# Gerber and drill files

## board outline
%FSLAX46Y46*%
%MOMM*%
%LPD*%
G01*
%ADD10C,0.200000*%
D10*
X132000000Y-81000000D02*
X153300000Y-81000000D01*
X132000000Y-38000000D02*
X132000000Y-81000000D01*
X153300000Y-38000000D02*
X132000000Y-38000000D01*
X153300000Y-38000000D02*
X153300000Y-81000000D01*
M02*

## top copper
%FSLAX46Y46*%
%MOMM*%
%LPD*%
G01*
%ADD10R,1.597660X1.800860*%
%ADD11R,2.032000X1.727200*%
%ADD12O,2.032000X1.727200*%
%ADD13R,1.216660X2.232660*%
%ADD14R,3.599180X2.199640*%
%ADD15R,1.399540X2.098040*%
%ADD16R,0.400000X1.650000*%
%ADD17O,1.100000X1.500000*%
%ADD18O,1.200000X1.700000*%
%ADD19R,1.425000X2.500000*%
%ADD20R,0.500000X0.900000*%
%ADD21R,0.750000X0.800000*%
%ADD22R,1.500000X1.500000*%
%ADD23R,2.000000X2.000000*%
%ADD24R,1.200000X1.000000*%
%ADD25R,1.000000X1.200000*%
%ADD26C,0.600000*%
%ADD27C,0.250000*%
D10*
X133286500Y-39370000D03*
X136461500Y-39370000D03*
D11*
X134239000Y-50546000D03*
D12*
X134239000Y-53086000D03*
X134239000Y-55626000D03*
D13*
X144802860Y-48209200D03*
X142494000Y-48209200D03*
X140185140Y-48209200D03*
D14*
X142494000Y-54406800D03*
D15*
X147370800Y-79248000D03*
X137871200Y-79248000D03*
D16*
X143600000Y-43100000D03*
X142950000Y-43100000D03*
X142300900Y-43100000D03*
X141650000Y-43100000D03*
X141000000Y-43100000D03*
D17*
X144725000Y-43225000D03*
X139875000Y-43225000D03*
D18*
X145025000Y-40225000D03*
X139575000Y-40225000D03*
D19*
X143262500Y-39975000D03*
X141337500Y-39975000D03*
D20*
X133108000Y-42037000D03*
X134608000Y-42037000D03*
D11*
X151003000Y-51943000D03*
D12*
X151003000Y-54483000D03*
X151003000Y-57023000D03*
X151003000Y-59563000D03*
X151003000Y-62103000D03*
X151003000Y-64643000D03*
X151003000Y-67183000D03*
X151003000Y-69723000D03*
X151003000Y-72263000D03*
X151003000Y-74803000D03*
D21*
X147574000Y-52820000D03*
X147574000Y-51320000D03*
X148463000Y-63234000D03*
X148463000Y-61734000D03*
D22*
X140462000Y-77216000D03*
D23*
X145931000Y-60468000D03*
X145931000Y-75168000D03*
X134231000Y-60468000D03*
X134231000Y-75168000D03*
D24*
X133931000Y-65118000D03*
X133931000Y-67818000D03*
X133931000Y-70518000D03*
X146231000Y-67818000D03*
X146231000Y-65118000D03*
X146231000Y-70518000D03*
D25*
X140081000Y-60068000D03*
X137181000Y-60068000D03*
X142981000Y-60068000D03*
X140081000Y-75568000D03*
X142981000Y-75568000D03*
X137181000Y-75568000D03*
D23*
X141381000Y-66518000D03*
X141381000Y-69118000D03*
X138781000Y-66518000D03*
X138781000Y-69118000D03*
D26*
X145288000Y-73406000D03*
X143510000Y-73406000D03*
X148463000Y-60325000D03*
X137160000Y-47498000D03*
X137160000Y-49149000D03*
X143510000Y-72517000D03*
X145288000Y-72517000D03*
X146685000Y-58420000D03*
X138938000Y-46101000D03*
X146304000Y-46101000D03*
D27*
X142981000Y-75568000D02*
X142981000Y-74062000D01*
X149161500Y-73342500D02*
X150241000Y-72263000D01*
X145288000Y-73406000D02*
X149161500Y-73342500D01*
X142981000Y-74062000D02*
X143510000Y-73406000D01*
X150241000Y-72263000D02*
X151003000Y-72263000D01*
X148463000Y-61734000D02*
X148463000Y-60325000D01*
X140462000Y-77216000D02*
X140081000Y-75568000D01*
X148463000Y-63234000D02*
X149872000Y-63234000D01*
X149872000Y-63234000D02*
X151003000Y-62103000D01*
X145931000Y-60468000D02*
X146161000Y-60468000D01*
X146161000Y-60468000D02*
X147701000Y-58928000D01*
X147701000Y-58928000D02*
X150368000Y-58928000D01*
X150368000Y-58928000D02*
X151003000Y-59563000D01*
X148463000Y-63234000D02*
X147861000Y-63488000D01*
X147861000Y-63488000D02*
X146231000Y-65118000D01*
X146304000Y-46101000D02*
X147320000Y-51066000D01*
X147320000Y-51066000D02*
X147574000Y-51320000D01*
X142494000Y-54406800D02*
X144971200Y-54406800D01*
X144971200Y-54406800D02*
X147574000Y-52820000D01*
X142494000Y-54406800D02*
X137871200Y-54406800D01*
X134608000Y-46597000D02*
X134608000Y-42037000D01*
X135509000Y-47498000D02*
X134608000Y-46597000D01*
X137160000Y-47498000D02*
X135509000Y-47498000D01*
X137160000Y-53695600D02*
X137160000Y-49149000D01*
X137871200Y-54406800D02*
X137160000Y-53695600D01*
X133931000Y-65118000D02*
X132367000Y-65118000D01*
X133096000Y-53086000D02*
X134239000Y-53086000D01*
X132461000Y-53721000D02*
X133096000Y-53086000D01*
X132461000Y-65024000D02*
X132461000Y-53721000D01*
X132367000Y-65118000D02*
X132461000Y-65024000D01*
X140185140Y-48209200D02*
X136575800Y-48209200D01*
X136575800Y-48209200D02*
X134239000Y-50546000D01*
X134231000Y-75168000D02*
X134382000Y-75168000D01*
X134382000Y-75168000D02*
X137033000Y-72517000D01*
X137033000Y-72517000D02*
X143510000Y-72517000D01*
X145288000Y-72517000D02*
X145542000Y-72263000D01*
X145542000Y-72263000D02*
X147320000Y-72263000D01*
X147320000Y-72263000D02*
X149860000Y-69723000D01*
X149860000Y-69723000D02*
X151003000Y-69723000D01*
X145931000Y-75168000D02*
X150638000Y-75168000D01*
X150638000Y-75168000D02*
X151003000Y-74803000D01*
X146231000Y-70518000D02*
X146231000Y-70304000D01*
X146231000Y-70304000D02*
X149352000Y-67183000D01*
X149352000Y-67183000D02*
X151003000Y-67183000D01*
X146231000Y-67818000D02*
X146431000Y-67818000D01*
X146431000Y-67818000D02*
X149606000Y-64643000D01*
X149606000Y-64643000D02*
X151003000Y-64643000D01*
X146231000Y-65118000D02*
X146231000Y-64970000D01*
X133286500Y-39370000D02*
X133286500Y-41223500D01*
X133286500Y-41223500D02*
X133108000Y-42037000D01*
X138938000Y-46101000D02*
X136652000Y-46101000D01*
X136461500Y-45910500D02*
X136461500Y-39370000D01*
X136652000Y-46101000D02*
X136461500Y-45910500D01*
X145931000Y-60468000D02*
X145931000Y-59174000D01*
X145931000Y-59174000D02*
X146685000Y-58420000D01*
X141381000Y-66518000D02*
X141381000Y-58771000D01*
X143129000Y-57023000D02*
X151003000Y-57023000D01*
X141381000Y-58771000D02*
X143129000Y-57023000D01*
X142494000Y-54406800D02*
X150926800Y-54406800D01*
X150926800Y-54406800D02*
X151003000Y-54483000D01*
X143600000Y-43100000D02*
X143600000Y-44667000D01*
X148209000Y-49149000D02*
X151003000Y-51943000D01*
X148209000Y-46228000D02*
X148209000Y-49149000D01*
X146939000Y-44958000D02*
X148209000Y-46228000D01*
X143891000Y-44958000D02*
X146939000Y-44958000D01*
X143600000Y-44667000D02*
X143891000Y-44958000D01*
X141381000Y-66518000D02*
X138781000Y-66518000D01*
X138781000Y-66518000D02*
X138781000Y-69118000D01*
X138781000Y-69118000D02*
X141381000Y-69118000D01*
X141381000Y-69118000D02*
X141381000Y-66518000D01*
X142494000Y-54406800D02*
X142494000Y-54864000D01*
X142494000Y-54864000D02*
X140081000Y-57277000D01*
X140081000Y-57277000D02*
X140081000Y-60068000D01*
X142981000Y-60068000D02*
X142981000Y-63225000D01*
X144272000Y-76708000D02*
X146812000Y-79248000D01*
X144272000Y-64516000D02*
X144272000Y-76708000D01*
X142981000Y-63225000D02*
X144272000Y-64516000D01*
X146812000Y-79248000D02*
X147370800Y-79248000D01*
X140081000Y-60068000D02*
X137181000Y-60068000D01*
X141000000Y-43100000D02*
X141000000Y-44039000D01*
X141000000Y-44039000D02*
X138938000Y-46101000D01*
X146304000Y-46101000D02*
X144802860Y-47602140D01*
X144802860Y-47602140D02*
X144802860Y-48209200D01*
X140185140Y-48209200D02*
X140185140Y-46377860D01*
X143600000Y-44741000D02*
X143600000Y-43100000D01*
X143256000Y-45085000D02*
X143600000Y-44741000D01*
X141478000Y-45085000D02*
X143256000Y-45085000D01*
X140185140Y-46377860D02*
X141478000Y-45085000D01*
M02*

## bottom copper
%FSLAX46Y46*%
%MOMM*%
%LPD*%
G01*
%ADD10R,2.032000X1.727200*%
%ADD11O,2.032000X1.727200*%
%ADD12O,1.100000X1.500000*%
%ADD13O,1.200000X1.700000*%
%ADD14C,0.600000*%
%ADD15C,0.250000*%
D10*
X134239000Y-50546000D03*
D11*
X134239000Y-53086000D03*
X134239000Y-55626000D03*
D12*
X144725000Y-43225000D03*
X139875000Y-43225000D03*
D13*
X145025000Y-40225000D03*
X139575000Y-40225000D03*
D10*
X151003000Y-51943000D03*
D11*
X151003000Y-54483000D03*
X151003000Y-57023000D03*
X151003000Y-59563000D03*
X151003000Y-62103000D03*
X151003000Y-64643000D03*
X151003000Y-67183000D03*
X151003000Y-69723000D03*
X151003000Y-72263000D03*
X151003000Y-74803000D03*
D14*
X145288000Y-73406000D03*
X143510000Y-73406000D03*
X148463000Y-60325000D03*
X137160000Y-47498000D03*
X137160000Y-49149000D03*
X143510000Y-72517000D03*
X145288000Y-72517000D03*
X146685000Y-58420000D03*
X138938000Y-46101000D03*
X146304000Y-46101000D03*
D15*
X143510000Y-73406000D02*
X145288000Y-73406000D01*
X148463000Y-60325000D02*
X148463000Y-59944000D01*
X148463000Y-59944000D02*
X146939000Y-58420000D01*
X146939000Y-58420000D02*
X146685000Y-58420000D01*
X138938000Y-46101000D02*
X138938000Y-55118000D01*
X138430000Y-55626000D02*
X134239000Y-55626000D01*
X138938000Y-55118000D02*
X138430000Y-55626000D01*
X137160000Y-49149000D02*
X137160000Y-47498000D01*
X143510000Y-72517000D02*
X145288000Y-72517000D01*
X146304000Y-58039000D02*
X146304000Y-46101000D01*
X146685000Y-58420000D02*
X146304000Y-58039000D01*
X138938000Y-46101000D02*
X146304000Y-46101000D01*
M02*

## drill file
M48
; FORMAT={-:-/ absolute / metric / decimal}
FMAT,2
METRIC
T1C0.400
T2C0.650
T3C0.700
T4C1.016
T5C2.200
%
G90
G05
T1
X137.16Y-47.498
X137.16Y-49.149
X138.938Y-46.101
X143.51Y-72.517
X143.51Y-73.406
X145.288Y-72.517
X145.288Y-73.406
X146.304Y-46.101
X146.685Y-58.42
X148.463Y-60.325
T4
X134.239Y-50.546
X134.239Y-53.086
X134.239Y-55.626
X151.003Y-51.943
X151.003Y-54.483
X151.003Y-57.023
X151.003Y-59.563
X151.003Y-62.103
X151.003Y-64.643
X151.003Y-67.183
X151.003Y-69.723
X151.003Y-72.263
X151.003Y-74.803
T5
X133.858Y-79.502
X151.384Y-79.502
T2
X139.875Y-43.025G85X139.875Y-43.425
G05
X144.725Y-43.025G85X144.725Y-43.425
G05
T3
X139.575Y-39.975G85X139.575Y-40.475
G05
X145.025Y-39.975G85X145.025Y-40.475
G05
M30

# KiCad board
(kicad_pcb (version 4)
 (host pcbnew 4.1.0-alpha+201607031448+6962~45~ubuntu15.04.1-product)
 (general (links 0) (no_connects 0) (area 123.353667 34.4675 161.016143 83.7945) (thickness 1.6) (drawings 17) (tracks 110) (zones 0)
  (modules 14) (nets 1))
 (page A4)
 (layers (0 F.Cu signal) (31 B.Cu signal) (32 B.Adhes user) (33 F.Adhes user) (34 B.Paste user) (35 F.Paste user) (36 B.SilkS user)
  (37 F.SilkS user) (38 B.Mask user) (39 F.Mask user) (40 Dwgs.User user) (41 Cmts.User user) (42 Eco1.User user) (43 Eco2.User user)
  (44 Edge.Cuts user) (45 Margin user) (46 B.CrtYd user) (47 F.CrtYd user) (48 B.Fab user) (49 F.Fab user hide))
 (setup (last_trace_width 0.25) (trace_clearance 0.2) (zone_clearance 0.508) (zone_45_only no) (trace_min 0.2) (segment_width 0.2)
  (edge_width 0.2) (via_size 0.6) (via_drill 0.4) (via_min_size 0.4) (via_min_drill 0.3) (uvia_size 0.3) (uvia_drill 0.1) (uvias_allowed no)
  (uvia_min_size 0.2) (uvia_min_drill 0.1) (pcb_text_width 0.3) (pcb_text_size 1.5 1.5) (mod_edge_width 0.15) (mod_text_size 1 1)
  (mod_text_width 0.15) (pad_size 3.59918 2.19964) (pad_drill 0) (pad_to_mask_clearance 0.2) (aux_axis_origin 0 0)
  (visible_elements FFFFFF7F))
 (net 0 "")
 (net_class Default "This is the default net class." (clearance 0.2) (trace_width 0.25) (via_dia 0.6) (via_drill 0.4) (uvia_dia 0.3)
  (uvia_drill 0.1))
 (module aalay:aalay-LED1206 (layer F.Cu) (at 134.874 39.37)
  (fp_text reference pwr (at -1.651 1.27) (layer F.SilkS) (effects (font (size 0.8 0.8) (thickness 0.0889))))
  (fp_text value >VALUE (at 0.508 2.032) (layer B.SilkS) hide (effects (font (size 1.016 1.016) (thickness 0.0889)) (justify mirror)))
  (pad A smd rect (at -1.5875 0) (size 1.59766 1.80086) (layers F.Cu F.Paste F.Mask))
  (pad K smd rect (at 1.5875 0) (size 1.59766 1.80086) (layers F.Cu F.Paste F.Mask)))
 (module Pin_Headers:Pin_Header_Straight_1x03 (layer F.Cu) (at 134.239 50.546)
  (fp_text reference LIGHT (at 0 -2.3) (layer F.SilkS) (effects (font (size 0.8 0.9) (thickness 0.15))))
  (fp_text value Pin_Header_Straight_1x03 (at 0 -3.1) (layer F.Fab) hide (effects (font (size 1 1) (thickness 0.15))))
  (pad 1 thru_hole rect (at 0 0) (size 2.032 1.7272) (drill 1.016) (layers *.Cu *.Mask F.SilkS))
  (pad 2 thru_hole oval (at 0 2.54) (size 2.032 1.7272) (drill 1.016) (layers *.Cu *.Mask F.SilkS))
  (pad 3 thru_hole oval (at 0 5.08) (size 2.032 1.7272) (drill 1.016) (layers *.Cu *.Mask F.SilkS)))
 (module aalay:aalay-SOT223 (layer F.Cu) (at 142.494 51.308 180)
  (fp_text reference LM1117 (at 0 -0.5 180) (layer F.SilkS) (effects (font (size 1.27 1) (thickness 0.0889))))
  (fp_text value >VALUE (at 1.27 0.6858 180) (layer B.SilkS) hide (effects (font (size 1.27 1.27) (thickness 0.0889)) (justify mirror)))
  (pad GND smd rect (at -2.30886 3.0988 180) (size 1.21666 2.23266) (layers F.Cu F.Paste F.Mask))
  (pad OUT smd rect (at 0 3.0988 180) (size 1.21666 2.23266) (layers F.Cu F.Paste F.Mask))
  (pad IN smd rect (at 2.30886 3.0988 180) (size 1.21666 2.23266) (layers F.Cu F.Paste F.Mask))
  (pad OUT smd rect (at 0 -3.0988 180) (size 3.59918 2.19964) (layers F.Cu F.Paste F.Mask)))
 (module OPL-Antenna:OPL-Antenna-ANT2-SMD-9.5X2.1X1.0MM (layer F.Cu) (at 142.621 79.248 180)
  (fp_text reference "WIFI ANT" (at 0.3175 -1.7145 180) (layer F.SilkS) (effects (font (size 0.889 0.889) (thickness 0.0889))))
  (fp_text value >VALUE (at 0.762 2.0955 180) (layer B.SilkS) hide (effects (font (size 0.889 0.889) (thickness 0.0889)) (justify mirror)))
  (pad 1 smd rect (at -4.7498 0 180) (size 1.39954 2.09804) (layers F.Cu F.Paste F.Mask))
  (pad 2 smd rect (at 4.7498 0 180) (size 1.39954 2.09804) (layers F.Cu F.Paste F.Mask)))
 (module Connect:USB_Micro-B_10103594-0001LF (layer F.Cu) (at 142.3 41.6 180)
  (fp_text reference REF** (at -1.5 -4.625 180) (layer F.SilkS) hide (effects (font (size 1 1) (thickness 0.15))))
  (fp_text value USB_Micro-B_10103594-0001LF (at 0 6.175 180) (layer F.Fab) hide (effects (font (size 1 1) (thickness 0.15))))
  (pad +5 smd rect (at -1.3 -1.5 270) (size 1.65 0.4) (layers F.Cu F.Paste F.Mask))
  (pad D- smd rect (at -0.65 -1.5 270) (size 1.65 0.4) (layers F.Cu F.Paste F.Mask))
  (pad D+ smd rect (at -0.0009 -1.5 270) (size 1.65 0.4) (layers F.Cu F.Paste F.Mask))
  (pad ID smd rect (at 0.65 -1.5 270) (size 1.65 0.4) (layers F.Cu F.Paste F.Mask))
  (pad GND smd rect (at 1.3 -1.5 270) (size 1.65 0.4) (layers F.Cu F.Paste F.Mask))
  (pad 6 thru_hole oval (at -2.425 -1.625 270) (size 1.5 1.1) (drill oval 1.05 0.65) (layers *.Cu *.Mask F.SilkS))
  (pad 6 thru_hole oval (at 2.425 -1.625 270) (size 1.5 1.1) (drill oval 1.05 0.65) (layers *.Cu *.Mask F.SilkS))
  (pad 6 thru_hole oval (at -2.725 1.375 270) (size 1.7 1.2) (drill oval 1.2 0.7) (layers *.Cu *.Mask F.SilkS))
  (pad 6 thru_hole oval (at 2.725 1.375 270) (size 1.7 1.2) (drill oval 1.2 0.7) (layers *.Cu *.Mask F.SilkS))
  (pad 6 smd rect (at -0.9625 1.625 270) (size 2.5 1.425) (layers F.Cu F.Paste F.Mask))
  (pad 6 smd rect (at 0.9625 1.625 270) (size 2.5 1.425) (layers F.Cu F.Paste F.Mask)))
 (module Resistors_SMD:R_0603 (layer F.Cu) (at 133.858 42.037)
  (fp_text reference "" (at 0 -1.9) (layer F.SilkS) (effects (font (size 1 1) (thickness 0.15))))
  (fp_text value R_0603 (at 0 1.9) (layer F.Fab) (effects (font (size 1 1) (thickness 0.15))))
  (pad 1 smd rect (at -0.75 0) (size 0.5 0.9) (layers F.Cu F.Paste F.Mask))
  (pad 2 smd rect (at 0.75 0) (size 0.5 0.9) (layers F.Cu F.Paste F.Mask)))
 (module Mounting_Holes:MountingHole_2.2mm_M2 (layer F.Cu) (at 133.858 79.502)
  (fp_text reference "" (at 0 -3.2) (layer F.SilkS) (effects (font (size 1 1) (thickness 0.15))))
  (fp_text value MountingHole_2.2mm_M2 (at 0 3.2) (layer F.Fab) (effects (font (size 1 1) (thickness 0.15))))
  (pad 1 np_thru_hole circle (at 0 0) (size 2.2 2.2) (drill 2.2) (layers *.Cu *.Mask F.SilkS)))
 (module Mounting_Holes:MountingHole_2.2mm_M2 (layer F.Cu) (at 151.384 79.502)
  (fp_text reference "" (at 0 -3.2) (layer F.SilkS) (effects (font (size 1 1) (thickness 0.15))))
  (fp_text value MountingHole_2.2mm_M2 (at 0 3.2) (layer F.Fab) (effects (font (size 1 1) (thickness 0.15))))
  (pad 1 np_thru_hole circle (at 0 0) (size 2.2 2.2) (drill 2.2) (layers *.Cu *.Mask F.SilkS)))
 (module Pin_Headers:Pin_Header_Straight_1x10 (layer F.Cu) (at 151.003 51.943)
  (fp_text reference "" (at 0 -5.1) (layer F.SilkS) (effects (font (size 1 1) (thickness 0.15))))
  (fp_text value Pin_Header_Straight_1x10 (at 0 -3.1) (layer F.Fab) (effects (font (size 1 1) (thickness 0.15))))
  (pad 1 thru_hole rect (at 0 0) (size 2.032 1.7272) (drill 1.016) (layers *.Cu *.Mask F.SilkS))
  (pad 2 thru_hole oval (at 0 2.54) (size 2.032 1.7272) (drill 1.016) (layers *.Cu *.Mask F.SilkS))
  (pad 3 thru_hole oval (at 0 5.08) (size 2.032 1.7272) (drill 1.016) (layers *.Cu *.Mask F.SilkS))
  (pad 4 thru_hole oval (at 0 7.62) (size 2.032 1.7272) (drill 1.016) (layers *.Cu *.Mask F.SilkS))
  (pad 5 thru_hole oval (at 0 10.16) (size 2.032 1.7272) (drill 1.016) (layers *.Cu *.Mask F.SilkS))
  (pad 6 thru_hole oval (at 0 12.7) (size 2.032 1.7272) (drill 1.016) (layers *.Cu *.Mask F.SilkS))
  (pad 7 thru_hole oval (at 0 15.24) (size 2.032 1.7272) (drill 1.016) (layers *.Cu *.Mask F.SilkS))
  (pad 8 thru_hole oval (at 0 17.78) (size 2.032 1.7272) (drill 1.016) (layers *.Cu *.Mask F.SilkS))
  (pad 9 thru_hole oval (at 0 20.32) (size 2.032 1.7272) (drill 1.016) (layers *.Cu *.Mask F.SilkS))
  (pad 10 thru_hole oval (at 0 22.86) (size 2.032 1.7272) (drill 1.016) (layers *.Cu *.Mask F.SilkS)))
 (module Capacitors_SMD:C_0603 (layer F.Cu) (at 147.574 52.07 90)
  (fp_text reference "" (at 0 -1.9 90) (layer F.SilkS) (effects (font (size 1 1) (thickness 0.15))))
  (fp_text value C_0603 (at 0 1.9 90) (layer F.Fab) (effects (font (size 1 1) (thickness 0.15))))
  (pad 1 smd rect (at -0.75 0 90) (size 0.8 0.75) (layers F.Cu F.Paste F.Mask))
  (pad 2 smd rect (at 0.75 0 90) (size 0.8 0.75) (layers F.Cu F.Paste F.Mask)))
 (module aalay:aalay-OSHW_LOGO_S (layer F.Cu) (at 150.368 44.831)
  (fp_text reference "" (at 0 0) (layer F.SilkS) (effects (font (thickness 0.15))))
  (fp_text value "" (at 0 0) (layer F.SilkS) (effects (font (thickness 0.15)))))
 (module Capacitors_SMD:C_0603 (layer F.Cu) (at 148.463 62.484 90)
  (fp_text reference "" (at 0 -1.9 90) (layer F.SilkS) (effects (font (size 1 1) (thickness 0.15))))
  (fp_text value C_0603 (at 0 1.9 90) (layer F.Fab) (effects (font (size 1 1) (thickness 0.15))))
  (pad 1 smd rect (at -0.75 0 90) (size 0.8 0.75) (layers F.Cu F.Paste F.Mask))
  (pad 2 smd rect (at 0.75 0 90) (size 0.8 0.75) (layers F.Cu F.Paste F.Mask)))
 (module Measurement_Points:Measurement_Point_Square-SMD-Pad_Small (layer F.Cu) (at 140.462 77.216)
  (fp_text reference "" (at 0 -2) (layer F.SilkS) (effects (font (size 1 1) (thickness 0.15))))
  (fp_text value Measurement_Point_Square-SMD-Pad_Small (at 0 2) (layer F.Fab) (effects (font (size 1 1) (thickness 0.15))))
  (pad 1 smd rect (at 0 0) (size 1.5 1.5) (layers F.Cu F.Mask)))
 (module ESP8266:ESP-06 (layer F.Cu) (at 140.081 67.818 270)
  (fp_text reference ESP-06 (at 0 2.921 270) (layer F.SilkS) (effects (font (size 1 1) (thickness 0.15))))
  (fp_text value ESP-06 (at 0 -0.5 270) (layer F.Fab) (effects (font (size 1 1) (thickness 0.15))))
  (pad GND smd rect (at -7.35 -5.85 270) (size 2 2) (layers F.Cu F.Paste F.Mask))
  (pad GP5 smd rect (at 7.35 -5.85 270) (size 2 2) (layers F.Cu F.Paste F.Mask))
  (pad GP16 smd rect (at -7.35 5.85 270) (size 2 2) (layers F.Cu F.Paste F.Mask))
  (pad GP15 smd rect (at 7.35 5.85 270) (size 2 2) (layers F.Cu F.Paste F.Mask))
  (pad GP14 smd rect (at -2.7 6.15 270) (size 1 1.2) (layers F.Cu F.Paste F.Mask))
  (pad GP12 smd rect (at 0 6.15 270) (size 1 1.2) (layers F.Cu F.Paste F.Mask))
  (pad GP13 smd rect (at 2.7 6.15 270) (size 1 1.2) (layers F.Cu F.Paste F.Mask))
  (pad TX smd rect (at 0 -6.15 270) (size 1 1.2) (layers F.Cu F.Paste F.Mask))
  (pad RST smd rect (at -2.7 -6.15 270) (size 1 1.2) (layers F.Cu F.Paste F.Mask))
  (pad RX smd rect (at 2.7 -6.15 270) (size 1 1.2) (layers F.Cu F.Paste F.Mask))
  (pad 3.3 smd rect (at -7.75 0 270) (size 1.2 1) (layers F.Cu F.Paste F.Mask))
  (pad CHPD smd rect (at -7.75 2.9 270) (size 1.2 1) (layers F.Cu F.Paste F.Mask))
  (pad ANT smd rect (at -7.75 -2.9 270) (size 1.2 1) (layers F.Cu F.Paste F.Mask))
  (pad GP2 smd rect (at 7.75 0 270) (size 1.2 1) (layers F.Cu F.Paste F.Mask))
  (pad GP0 smd rect (at 7.75 -2.9 270) (size 1.2 1) (layers F.Cu F.Paste F.Mask))
  (pad GP4 smd rect (at 7.75 2.9 270) (size 1.2 1) (layers F.Cu F.Paste F.Mask))
  (pad GND smd rect (at -1.3 -1.3 270) (size 2 2) (layers F.Cu F.Paste F.Mask))
  (pad GND smd rect (at 1.3 -1.3 270) (size 2 2) (layers F.Cu F.Paste F.Mask))
  (pad GND smd rect (at -1.3 1.3 270) (size 2 2) (layers F.Cu F.Paste F.Mask))
  (pad GND smd rect (at 1.3 1.3 270) (size 2 2) (layers F.Cu F.Paste F.Mask)))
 (gr_line (start 132 81) (end 153.3 81) (angle 90) (layer Edge.Cuts) (width 0.2))
 (gr_line (start 132 38) (end 132 81) (angle 90) (layer Edge.Cuts) (width 0.2))
 (gr_line (start 153.3 38) (end 132 38) (angle 90) (layer Edge.Cuts) (width 0.2))
 (gr_line (start 153.3 38) (end 153.3 81) (angle 90) (layer Edge.Cuts) (width 0.2))
 (segment (start 142.981 75.568) (end 142.981 74.062) (width 0.25) (layer F.Cu) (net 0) (status 400000))
 (segment (start 149.1615 73.3425) (end 150.241 72.263) (width 0.25) (layer F.Cu) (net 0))
 (segment (start 145.288 73.406) (end 149.1615 73.3425) (width 0.25) (layer F.Cu) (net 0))
 (via (at 145.288 73.406) (size 0.6) (drill 0.4) (layers F.Cu B.Cu) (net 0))
 (segment (start 143.51 73.406) (end 145.288 73.406) (width 0.25) (layer B.Cu) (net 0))
 (via (at 143.51 73.406) (size 0.6) (drill 0.4) (layers F.Cu B.Cu) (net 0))
 (segment (start 142.981 74.062) (end 143.51 73.406) (width 0.25) (layer F.Cu) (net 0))
 (segment (start 150.241 72.263) (end 151.003 72.263) (width 0.25) (layer F.Cu) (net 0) (status C00000))
 (segment (start 148.463 61.734) (end 148.463 60.325) (width 0.25) (layer F.Cu) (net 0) (status 10))
 (via (at 148.463 60.325) (size 0.6) (drill 0.4) (layers F.Cu B.Cu) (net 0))
 (segment (start 148.463 60.325) (end 148.463 59.944) (width 0.25) (layer B.Cu) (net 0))
 (segment (start 148.463 59.944) (end 146.939 58.42) (width 0.25) (layer B.Cu) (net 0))
 (segment (start 146.939 58.42) (end 146.685 58.42) (width 0.25) (layer B.Cu) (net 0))
 (segment (start 140.462 77.216) (end 140.081 75.568) (width 0.25) (layer F.Cu) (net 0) (status 10))
 (segment (start 148.463 63.234) (end 149.872 63.234) (width 0.25) (layer F.Cu) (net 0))
 (segment (start 149.872 63.234) (end 151.003 62.103) (width 0.25) (layer F.Cu) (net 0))
 (segment (start 145.931 60.468) (end 146.161 60.468) (width 0.25) (layer F.Cu) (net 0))
 (segment (start 146.161 60.468) (end 147.701 58.928) (width 0.25) (layer F.Cu) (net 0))
 (segment (start 147.701 58.928) (end 150.368 58.928) (width 0.25) (layer F.Cu) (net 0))
 (segment (start 150.368 58.928) (end 151.003 59.563) (width 0.25) (layer F.Cu) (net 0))
 (segment (start 148.463 63.234) (end 147.861 63.488) (width 0.25) (layer F.Cu) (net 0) (status 10))
 (segment (start 147.861 63.488) (end 146.231 65.118) (width 0.25) (layer F.Cu) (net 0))
 (segment (start 146.304 46.101) (end 147.32 51.066) (width 0.25) (layer F.Cu) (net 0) (status 20))
 (segment (start 147.32 51.066) (end 147.574 51.32) (width 0.25) (layer F.Cu) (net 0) (status 30))
 (segment (start 142.494 54.4068) (end 144.9712 54.4068) (width 0.25) (layer F.Cu) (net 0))
 (segment (start 144.9712 54.4068) (end 147.574 52.82) (width 0.25) (layer F.Cu) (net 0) (status 20))
 (segment (start 138.938 46.101) (end 138.938 55.118) (width 0.25) (layer B.Cu) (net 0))
 (segment (start 138.43 55.626) (end 134.239 55.626) (width 0.25) (layer B.Cu) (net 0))
 (segment (start 138.938 55.118) (end 138.43 55.626) (width 0.25) (layer B.Cu) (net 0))
 (segment (start 142.494 54.4068) (end 137.8712 54.4068) (width 0.25) (layer F.Cu) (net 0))
 (segment (start 134.608 46.597) (end 134.608 42.037) (width 0.25) (layer F.Cu) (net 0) (status 20))
 (segment (start 135.509 47.498) (end 134.608 46.597) (width 0.25) (layer F.Cu) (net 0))
 (segment (start 137.16 47.498) (end 135.509 47.498) (width 0.25) (layer F.Cu) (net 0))
 (via (at 137.16 47.498) (size 0.6) (drill 0.4) (layers F.Cu B.Cu) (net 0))
 (segment (start 137.16 49.149) (end 137.16 47.498) (width 0.25) (layer B.Cu) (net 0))
 (via (at 137.16 49.149) (size 0.6) (drill 0.4) (layers F.Cu B.Cu) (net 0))
 (segment (start 137.16 53.6956) (end 137.16 49.149) (width 0.25) (layer F.Cu) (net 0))
 (segment (start 137.8712 54.4068) (end 137.16 53.6956) (width 0.25) (layer F.Cu) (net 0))
 (segment (start 133.931 65.118) (end 132.367 65.118) (width 0.25) (layer F.Cu) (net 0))
 (segment (start 133.096 53.086) (end 134.239 53.086) (width 0.25) (layer F.Cu) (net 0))
 (segment (start 132.461 53.721) (end 133.096 53.086) (width 0.25) (layer F.Cu) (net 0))
 (segment (start 132.461 65.024) (end 132.461 53.721) (width 0.25) (layer F.Cu) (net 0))
 (segment (start 132.367 65.118) (end 132.461 65.024) (width 0.25) (layer F.Cu) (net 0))
 (segment (start 140.18514 48.2092) (end 136.5758 48.2092) (width 0.25) (layer F.Cu) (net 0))
 (segment (start 136.5758 48.2092) (end 134.239 50.546) (width 0.25) (layer F.Cu) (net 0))
 (segment (start 134.231 75.168) (end 134.382 75.168) (width 0.25) (layer F.Cu) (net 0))
 (segment (start 134.382 75.168) (end 137.033 72.517) (width 0.25) (layer F.Cu) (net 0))
 (segment (start 137.033 72.517) (end 143.51 72.517) (width 0.25) (layer F.Cu) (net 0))
 (via (at 143.51 72.517) (size 0.6) (drill 0.4) (layers F.Cu B.Cu) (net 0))
 (segment (start 143.51 72.517) (end 145.288 72.517) (width 0.25) (layer B.Cu) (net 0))
 (via (at 145.288 72.517) (size 0.6) (drill 0.4) (layers F.Cu B.Cu) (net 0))
 (segment (start 145.288 72.517) (end 145.542 72.263) (width 0.25) (layer F.Cu) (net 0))
 (segment (start 145.542 72.263) (end 147.32 72.263) (width 0.25) (layer F.Cu) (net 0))
 (segment (start 147.32 72.263) (end 149.86 69.723) (width 0.25) (layer F.Cu) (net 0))
 (segment (start 149.86 69.723) (end 151.003 69.723) (width 0.25) (layer F.Cu) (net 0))
 (segment (start 145.931 75.168) (end 150.638 75.168) (width 0.25) (layer F.Cu) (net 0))
 (segment (start 150.638 75.168) (end 151.003 74.803) (width 0.25) (layer F.Cu) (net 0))
 (segment (start 146.231 70.518) (end 146.231 70.304) (width 0.25) (layer F.Cu) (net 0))
 (segment (start 146.231 70.304) (end 149.352 67.183) (width 0.25) (layer F.Cu) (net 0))
 (segment (start 149.352 67.183) (end 151.003 67.183) (width 0.25) (layer F.Cu) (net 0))
 (segment (start 146.231 67.818) (end 146.431 67.818) (width 0.25) (layer F.Cu) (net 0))
 (segment (start 146.431 67.818) (end 149.606 64.643) (width 0.25) (layer F.Cu) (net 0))
 (segment (start 149.606 64.643) (end 151.003 64.643) (width 0.25) (layer F.Cu) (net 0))
 (segment (start 146.231 65.118) (end 146.231 64.97) (width 0.25) (layer F.Cu) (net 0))
 (segment (start 133.2865 39.37) (end 133.2865 41.2235) (width 0.25) (layer F.Cu) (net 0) (status 10))
 (segment (start 133.2865 41.2235) (end 133.108 42.037) (width 0.25) (layer F.Cu) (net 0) (status 20))
 (segment (start 138.938 46.101) (end 136.652 46.101) (width 0.25) (layer F.Cu) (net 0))
 (segment (start 136.4615 45.9105) (end 136.4615 39.37) (width 0.25) (layer F.Cu) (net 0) (status 20))
 (segment (start 136.652 46.101) (end 136.4615 45.9105) (width 0.25) (layer F.Cu) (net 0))
 (segment (start 145.931 60.468) (end 145.931 59.174) (width 0.25) (layer F.Cu) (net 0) (status 10))
 (segment (start 146.304 58.039) (end 146.304 46.101) (width 0.25) (layer B.Cu) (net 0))
 (segment (start 146.685 58.42) (end 146.304 58.039) (width 0.25) (layer B.Cu) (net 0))
 (via (at 146.685 58.42) (size 0.6) (drill 0.4) (layers F.Cu B.Cu) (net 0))
 (segment (start 145.931 59.174) (end 146.685 58.42) (width 0.25) (layer F.Cu) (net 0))
 (segment (start 141.381 66.518) (end 141.381 58.771) (width 0.25) (layer F.Cu) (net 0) (status 10))
 (segment (start 143.129 57.023) (end 151.003 57.023) (width 0.25) (layer F.Cu) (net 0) (status 20))
 (segment (start 141.381 58.771) (end 143.129 57.023) (width 0.25) (layer F.Cu) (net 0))
 (segment (start 142.494 54.4068) (end 150.9268 54.4068) (width 0.25) (layer F.Cu) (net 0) (status 30))
 (segment (start 150.9268 54.4068) (end 151.003 54.483) (width 0.25) (layer F.Cu) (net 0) (status 30))
 (segment (start 143.6 43.1) (end 143.6 44.667) (width 0.25) (layer F.Cu) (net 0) (status 10))
 (segment (start 148.209 49.149) (end 151.003 51.943) (width 0.25) (layer F.Cu) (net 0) (status 20))
 (segment (start 148.209 46.228) (end 148.209 49.149) (width 0.25) (layer F.Cu) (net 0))
 (segment (start 146.939 44.958) (end 148.209 46.228) (width 0.25) (layer F.Cu) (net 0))
 (segment (start 143.891 44.958) (end 146.939 44.958) (width 0.25) (layer F.Cu) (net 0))
 (segment (start 143.6 44.667) (end 143.891 44.958) (width 0.25) (layer F.Cu) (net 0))
 (segment (start 141.381 66.518) (end 138.781 66.518) (width 0.25) (layer F.Cu) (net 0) (status 30))
 (segment (start 138.781 66.518) (end 138.781 69.118) (width 0.25) (layer F.Cu) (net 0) (status 30))
 (segment (start 138.781 69.118) (end 141.381 69.118) (width 0.25) (layer F.Cu) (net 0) (status 30))
 (segment (start 141.381 69.118) (end 141.381 66.518) (width 0.25) (layer F.Cu) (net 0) (status 30))
 (segment (start 142.494 54.4068) (end 142.494 54.864) (width 0.25) (layer F.Cu) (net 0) (status 30))
 (segment (start 142.494 54.864) (end 140.081 57.277) (width 0.25) (layer F.Cu) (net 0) (status 10))
 (segment (start 140.081 57.277) (end 140.081 60.068) (width 0.25) (layer F.Cu) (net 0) (status 20))
 (segment (start 142.981 60.068) (end 142.981 63.225) (width 0.25) (layer F.Cu) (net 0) (status 10))
 (segment (start 144.272 76.708) (end 146.812 79.248) (width 0.25) (layer F.Cu) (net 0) (status 20))
 (segment (start 144.272 64.516) (end 144.272 76.708) (width 0.25) (layer F.Cu) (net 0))
 (segment (start 142.981 63.225) (end 144.272 64.516) (width 0.25) (layer F.Cu) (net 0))
 (segment (start 146.812 79.248) (end 147.3708 79.248) (width 0.25) (layer F.Cu) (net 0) (status 30))
 (segment (start 140.081 60.068) (end 137.181 60.068) (width 0.25) (layer F.Cu) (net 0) (status 30))
 (segment (start 141 43.1) (end 141 44.039) (width 0.25) (layer F.Cu) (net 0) (status 10))
 (segment (start 141 44.039) (end 138.938 46.101) (width 0.25) (layer F.Cu) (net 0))
 (via (at 138.938 46.101) (size 0.6) (drill 0.4) (layers F.Cu B.Cu) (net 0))
 (segment (start 138.938 46.101) (end 146.304 46.101) (width 0.25) (layer B.Cu) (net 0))
 (segment (start 146.304 46.101) (end 144.80286 47.60214) (width 0.25) (layer F.Cu) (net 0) (status 20))
 (via (at 146.304 46.101) (size 0.6) (drill 0.4) (layers F.Cu B.Cu) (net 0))
 (segment (start 144.80286 47.60214) (end 144.80286 48.2092) (width 0.25) (layer F.Cu) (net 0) (status 30))
 (segment (start 140.18514 48.2092) (end 140.18514 46.37786) (width 0.25) (layer F.Cu) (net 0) (status 10))
 (segment (start 143.6 44.741) (end 143.6 43.1) (width 0.25) (layer F.Cu) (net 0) (status 20))
 (segment (start 143.256 45.085) (end 143.6 44.741) (width 0.25) (layer F.Cu) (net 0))
 (segment (start 141.478 45.085) (end 143.256 45.085) (width 0.25) (layer F.Cu) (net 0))
 (segment (start 140.18514 46.37786) (end 141.478 45.085) (width 0.25) (layer F.Cu) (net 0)))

